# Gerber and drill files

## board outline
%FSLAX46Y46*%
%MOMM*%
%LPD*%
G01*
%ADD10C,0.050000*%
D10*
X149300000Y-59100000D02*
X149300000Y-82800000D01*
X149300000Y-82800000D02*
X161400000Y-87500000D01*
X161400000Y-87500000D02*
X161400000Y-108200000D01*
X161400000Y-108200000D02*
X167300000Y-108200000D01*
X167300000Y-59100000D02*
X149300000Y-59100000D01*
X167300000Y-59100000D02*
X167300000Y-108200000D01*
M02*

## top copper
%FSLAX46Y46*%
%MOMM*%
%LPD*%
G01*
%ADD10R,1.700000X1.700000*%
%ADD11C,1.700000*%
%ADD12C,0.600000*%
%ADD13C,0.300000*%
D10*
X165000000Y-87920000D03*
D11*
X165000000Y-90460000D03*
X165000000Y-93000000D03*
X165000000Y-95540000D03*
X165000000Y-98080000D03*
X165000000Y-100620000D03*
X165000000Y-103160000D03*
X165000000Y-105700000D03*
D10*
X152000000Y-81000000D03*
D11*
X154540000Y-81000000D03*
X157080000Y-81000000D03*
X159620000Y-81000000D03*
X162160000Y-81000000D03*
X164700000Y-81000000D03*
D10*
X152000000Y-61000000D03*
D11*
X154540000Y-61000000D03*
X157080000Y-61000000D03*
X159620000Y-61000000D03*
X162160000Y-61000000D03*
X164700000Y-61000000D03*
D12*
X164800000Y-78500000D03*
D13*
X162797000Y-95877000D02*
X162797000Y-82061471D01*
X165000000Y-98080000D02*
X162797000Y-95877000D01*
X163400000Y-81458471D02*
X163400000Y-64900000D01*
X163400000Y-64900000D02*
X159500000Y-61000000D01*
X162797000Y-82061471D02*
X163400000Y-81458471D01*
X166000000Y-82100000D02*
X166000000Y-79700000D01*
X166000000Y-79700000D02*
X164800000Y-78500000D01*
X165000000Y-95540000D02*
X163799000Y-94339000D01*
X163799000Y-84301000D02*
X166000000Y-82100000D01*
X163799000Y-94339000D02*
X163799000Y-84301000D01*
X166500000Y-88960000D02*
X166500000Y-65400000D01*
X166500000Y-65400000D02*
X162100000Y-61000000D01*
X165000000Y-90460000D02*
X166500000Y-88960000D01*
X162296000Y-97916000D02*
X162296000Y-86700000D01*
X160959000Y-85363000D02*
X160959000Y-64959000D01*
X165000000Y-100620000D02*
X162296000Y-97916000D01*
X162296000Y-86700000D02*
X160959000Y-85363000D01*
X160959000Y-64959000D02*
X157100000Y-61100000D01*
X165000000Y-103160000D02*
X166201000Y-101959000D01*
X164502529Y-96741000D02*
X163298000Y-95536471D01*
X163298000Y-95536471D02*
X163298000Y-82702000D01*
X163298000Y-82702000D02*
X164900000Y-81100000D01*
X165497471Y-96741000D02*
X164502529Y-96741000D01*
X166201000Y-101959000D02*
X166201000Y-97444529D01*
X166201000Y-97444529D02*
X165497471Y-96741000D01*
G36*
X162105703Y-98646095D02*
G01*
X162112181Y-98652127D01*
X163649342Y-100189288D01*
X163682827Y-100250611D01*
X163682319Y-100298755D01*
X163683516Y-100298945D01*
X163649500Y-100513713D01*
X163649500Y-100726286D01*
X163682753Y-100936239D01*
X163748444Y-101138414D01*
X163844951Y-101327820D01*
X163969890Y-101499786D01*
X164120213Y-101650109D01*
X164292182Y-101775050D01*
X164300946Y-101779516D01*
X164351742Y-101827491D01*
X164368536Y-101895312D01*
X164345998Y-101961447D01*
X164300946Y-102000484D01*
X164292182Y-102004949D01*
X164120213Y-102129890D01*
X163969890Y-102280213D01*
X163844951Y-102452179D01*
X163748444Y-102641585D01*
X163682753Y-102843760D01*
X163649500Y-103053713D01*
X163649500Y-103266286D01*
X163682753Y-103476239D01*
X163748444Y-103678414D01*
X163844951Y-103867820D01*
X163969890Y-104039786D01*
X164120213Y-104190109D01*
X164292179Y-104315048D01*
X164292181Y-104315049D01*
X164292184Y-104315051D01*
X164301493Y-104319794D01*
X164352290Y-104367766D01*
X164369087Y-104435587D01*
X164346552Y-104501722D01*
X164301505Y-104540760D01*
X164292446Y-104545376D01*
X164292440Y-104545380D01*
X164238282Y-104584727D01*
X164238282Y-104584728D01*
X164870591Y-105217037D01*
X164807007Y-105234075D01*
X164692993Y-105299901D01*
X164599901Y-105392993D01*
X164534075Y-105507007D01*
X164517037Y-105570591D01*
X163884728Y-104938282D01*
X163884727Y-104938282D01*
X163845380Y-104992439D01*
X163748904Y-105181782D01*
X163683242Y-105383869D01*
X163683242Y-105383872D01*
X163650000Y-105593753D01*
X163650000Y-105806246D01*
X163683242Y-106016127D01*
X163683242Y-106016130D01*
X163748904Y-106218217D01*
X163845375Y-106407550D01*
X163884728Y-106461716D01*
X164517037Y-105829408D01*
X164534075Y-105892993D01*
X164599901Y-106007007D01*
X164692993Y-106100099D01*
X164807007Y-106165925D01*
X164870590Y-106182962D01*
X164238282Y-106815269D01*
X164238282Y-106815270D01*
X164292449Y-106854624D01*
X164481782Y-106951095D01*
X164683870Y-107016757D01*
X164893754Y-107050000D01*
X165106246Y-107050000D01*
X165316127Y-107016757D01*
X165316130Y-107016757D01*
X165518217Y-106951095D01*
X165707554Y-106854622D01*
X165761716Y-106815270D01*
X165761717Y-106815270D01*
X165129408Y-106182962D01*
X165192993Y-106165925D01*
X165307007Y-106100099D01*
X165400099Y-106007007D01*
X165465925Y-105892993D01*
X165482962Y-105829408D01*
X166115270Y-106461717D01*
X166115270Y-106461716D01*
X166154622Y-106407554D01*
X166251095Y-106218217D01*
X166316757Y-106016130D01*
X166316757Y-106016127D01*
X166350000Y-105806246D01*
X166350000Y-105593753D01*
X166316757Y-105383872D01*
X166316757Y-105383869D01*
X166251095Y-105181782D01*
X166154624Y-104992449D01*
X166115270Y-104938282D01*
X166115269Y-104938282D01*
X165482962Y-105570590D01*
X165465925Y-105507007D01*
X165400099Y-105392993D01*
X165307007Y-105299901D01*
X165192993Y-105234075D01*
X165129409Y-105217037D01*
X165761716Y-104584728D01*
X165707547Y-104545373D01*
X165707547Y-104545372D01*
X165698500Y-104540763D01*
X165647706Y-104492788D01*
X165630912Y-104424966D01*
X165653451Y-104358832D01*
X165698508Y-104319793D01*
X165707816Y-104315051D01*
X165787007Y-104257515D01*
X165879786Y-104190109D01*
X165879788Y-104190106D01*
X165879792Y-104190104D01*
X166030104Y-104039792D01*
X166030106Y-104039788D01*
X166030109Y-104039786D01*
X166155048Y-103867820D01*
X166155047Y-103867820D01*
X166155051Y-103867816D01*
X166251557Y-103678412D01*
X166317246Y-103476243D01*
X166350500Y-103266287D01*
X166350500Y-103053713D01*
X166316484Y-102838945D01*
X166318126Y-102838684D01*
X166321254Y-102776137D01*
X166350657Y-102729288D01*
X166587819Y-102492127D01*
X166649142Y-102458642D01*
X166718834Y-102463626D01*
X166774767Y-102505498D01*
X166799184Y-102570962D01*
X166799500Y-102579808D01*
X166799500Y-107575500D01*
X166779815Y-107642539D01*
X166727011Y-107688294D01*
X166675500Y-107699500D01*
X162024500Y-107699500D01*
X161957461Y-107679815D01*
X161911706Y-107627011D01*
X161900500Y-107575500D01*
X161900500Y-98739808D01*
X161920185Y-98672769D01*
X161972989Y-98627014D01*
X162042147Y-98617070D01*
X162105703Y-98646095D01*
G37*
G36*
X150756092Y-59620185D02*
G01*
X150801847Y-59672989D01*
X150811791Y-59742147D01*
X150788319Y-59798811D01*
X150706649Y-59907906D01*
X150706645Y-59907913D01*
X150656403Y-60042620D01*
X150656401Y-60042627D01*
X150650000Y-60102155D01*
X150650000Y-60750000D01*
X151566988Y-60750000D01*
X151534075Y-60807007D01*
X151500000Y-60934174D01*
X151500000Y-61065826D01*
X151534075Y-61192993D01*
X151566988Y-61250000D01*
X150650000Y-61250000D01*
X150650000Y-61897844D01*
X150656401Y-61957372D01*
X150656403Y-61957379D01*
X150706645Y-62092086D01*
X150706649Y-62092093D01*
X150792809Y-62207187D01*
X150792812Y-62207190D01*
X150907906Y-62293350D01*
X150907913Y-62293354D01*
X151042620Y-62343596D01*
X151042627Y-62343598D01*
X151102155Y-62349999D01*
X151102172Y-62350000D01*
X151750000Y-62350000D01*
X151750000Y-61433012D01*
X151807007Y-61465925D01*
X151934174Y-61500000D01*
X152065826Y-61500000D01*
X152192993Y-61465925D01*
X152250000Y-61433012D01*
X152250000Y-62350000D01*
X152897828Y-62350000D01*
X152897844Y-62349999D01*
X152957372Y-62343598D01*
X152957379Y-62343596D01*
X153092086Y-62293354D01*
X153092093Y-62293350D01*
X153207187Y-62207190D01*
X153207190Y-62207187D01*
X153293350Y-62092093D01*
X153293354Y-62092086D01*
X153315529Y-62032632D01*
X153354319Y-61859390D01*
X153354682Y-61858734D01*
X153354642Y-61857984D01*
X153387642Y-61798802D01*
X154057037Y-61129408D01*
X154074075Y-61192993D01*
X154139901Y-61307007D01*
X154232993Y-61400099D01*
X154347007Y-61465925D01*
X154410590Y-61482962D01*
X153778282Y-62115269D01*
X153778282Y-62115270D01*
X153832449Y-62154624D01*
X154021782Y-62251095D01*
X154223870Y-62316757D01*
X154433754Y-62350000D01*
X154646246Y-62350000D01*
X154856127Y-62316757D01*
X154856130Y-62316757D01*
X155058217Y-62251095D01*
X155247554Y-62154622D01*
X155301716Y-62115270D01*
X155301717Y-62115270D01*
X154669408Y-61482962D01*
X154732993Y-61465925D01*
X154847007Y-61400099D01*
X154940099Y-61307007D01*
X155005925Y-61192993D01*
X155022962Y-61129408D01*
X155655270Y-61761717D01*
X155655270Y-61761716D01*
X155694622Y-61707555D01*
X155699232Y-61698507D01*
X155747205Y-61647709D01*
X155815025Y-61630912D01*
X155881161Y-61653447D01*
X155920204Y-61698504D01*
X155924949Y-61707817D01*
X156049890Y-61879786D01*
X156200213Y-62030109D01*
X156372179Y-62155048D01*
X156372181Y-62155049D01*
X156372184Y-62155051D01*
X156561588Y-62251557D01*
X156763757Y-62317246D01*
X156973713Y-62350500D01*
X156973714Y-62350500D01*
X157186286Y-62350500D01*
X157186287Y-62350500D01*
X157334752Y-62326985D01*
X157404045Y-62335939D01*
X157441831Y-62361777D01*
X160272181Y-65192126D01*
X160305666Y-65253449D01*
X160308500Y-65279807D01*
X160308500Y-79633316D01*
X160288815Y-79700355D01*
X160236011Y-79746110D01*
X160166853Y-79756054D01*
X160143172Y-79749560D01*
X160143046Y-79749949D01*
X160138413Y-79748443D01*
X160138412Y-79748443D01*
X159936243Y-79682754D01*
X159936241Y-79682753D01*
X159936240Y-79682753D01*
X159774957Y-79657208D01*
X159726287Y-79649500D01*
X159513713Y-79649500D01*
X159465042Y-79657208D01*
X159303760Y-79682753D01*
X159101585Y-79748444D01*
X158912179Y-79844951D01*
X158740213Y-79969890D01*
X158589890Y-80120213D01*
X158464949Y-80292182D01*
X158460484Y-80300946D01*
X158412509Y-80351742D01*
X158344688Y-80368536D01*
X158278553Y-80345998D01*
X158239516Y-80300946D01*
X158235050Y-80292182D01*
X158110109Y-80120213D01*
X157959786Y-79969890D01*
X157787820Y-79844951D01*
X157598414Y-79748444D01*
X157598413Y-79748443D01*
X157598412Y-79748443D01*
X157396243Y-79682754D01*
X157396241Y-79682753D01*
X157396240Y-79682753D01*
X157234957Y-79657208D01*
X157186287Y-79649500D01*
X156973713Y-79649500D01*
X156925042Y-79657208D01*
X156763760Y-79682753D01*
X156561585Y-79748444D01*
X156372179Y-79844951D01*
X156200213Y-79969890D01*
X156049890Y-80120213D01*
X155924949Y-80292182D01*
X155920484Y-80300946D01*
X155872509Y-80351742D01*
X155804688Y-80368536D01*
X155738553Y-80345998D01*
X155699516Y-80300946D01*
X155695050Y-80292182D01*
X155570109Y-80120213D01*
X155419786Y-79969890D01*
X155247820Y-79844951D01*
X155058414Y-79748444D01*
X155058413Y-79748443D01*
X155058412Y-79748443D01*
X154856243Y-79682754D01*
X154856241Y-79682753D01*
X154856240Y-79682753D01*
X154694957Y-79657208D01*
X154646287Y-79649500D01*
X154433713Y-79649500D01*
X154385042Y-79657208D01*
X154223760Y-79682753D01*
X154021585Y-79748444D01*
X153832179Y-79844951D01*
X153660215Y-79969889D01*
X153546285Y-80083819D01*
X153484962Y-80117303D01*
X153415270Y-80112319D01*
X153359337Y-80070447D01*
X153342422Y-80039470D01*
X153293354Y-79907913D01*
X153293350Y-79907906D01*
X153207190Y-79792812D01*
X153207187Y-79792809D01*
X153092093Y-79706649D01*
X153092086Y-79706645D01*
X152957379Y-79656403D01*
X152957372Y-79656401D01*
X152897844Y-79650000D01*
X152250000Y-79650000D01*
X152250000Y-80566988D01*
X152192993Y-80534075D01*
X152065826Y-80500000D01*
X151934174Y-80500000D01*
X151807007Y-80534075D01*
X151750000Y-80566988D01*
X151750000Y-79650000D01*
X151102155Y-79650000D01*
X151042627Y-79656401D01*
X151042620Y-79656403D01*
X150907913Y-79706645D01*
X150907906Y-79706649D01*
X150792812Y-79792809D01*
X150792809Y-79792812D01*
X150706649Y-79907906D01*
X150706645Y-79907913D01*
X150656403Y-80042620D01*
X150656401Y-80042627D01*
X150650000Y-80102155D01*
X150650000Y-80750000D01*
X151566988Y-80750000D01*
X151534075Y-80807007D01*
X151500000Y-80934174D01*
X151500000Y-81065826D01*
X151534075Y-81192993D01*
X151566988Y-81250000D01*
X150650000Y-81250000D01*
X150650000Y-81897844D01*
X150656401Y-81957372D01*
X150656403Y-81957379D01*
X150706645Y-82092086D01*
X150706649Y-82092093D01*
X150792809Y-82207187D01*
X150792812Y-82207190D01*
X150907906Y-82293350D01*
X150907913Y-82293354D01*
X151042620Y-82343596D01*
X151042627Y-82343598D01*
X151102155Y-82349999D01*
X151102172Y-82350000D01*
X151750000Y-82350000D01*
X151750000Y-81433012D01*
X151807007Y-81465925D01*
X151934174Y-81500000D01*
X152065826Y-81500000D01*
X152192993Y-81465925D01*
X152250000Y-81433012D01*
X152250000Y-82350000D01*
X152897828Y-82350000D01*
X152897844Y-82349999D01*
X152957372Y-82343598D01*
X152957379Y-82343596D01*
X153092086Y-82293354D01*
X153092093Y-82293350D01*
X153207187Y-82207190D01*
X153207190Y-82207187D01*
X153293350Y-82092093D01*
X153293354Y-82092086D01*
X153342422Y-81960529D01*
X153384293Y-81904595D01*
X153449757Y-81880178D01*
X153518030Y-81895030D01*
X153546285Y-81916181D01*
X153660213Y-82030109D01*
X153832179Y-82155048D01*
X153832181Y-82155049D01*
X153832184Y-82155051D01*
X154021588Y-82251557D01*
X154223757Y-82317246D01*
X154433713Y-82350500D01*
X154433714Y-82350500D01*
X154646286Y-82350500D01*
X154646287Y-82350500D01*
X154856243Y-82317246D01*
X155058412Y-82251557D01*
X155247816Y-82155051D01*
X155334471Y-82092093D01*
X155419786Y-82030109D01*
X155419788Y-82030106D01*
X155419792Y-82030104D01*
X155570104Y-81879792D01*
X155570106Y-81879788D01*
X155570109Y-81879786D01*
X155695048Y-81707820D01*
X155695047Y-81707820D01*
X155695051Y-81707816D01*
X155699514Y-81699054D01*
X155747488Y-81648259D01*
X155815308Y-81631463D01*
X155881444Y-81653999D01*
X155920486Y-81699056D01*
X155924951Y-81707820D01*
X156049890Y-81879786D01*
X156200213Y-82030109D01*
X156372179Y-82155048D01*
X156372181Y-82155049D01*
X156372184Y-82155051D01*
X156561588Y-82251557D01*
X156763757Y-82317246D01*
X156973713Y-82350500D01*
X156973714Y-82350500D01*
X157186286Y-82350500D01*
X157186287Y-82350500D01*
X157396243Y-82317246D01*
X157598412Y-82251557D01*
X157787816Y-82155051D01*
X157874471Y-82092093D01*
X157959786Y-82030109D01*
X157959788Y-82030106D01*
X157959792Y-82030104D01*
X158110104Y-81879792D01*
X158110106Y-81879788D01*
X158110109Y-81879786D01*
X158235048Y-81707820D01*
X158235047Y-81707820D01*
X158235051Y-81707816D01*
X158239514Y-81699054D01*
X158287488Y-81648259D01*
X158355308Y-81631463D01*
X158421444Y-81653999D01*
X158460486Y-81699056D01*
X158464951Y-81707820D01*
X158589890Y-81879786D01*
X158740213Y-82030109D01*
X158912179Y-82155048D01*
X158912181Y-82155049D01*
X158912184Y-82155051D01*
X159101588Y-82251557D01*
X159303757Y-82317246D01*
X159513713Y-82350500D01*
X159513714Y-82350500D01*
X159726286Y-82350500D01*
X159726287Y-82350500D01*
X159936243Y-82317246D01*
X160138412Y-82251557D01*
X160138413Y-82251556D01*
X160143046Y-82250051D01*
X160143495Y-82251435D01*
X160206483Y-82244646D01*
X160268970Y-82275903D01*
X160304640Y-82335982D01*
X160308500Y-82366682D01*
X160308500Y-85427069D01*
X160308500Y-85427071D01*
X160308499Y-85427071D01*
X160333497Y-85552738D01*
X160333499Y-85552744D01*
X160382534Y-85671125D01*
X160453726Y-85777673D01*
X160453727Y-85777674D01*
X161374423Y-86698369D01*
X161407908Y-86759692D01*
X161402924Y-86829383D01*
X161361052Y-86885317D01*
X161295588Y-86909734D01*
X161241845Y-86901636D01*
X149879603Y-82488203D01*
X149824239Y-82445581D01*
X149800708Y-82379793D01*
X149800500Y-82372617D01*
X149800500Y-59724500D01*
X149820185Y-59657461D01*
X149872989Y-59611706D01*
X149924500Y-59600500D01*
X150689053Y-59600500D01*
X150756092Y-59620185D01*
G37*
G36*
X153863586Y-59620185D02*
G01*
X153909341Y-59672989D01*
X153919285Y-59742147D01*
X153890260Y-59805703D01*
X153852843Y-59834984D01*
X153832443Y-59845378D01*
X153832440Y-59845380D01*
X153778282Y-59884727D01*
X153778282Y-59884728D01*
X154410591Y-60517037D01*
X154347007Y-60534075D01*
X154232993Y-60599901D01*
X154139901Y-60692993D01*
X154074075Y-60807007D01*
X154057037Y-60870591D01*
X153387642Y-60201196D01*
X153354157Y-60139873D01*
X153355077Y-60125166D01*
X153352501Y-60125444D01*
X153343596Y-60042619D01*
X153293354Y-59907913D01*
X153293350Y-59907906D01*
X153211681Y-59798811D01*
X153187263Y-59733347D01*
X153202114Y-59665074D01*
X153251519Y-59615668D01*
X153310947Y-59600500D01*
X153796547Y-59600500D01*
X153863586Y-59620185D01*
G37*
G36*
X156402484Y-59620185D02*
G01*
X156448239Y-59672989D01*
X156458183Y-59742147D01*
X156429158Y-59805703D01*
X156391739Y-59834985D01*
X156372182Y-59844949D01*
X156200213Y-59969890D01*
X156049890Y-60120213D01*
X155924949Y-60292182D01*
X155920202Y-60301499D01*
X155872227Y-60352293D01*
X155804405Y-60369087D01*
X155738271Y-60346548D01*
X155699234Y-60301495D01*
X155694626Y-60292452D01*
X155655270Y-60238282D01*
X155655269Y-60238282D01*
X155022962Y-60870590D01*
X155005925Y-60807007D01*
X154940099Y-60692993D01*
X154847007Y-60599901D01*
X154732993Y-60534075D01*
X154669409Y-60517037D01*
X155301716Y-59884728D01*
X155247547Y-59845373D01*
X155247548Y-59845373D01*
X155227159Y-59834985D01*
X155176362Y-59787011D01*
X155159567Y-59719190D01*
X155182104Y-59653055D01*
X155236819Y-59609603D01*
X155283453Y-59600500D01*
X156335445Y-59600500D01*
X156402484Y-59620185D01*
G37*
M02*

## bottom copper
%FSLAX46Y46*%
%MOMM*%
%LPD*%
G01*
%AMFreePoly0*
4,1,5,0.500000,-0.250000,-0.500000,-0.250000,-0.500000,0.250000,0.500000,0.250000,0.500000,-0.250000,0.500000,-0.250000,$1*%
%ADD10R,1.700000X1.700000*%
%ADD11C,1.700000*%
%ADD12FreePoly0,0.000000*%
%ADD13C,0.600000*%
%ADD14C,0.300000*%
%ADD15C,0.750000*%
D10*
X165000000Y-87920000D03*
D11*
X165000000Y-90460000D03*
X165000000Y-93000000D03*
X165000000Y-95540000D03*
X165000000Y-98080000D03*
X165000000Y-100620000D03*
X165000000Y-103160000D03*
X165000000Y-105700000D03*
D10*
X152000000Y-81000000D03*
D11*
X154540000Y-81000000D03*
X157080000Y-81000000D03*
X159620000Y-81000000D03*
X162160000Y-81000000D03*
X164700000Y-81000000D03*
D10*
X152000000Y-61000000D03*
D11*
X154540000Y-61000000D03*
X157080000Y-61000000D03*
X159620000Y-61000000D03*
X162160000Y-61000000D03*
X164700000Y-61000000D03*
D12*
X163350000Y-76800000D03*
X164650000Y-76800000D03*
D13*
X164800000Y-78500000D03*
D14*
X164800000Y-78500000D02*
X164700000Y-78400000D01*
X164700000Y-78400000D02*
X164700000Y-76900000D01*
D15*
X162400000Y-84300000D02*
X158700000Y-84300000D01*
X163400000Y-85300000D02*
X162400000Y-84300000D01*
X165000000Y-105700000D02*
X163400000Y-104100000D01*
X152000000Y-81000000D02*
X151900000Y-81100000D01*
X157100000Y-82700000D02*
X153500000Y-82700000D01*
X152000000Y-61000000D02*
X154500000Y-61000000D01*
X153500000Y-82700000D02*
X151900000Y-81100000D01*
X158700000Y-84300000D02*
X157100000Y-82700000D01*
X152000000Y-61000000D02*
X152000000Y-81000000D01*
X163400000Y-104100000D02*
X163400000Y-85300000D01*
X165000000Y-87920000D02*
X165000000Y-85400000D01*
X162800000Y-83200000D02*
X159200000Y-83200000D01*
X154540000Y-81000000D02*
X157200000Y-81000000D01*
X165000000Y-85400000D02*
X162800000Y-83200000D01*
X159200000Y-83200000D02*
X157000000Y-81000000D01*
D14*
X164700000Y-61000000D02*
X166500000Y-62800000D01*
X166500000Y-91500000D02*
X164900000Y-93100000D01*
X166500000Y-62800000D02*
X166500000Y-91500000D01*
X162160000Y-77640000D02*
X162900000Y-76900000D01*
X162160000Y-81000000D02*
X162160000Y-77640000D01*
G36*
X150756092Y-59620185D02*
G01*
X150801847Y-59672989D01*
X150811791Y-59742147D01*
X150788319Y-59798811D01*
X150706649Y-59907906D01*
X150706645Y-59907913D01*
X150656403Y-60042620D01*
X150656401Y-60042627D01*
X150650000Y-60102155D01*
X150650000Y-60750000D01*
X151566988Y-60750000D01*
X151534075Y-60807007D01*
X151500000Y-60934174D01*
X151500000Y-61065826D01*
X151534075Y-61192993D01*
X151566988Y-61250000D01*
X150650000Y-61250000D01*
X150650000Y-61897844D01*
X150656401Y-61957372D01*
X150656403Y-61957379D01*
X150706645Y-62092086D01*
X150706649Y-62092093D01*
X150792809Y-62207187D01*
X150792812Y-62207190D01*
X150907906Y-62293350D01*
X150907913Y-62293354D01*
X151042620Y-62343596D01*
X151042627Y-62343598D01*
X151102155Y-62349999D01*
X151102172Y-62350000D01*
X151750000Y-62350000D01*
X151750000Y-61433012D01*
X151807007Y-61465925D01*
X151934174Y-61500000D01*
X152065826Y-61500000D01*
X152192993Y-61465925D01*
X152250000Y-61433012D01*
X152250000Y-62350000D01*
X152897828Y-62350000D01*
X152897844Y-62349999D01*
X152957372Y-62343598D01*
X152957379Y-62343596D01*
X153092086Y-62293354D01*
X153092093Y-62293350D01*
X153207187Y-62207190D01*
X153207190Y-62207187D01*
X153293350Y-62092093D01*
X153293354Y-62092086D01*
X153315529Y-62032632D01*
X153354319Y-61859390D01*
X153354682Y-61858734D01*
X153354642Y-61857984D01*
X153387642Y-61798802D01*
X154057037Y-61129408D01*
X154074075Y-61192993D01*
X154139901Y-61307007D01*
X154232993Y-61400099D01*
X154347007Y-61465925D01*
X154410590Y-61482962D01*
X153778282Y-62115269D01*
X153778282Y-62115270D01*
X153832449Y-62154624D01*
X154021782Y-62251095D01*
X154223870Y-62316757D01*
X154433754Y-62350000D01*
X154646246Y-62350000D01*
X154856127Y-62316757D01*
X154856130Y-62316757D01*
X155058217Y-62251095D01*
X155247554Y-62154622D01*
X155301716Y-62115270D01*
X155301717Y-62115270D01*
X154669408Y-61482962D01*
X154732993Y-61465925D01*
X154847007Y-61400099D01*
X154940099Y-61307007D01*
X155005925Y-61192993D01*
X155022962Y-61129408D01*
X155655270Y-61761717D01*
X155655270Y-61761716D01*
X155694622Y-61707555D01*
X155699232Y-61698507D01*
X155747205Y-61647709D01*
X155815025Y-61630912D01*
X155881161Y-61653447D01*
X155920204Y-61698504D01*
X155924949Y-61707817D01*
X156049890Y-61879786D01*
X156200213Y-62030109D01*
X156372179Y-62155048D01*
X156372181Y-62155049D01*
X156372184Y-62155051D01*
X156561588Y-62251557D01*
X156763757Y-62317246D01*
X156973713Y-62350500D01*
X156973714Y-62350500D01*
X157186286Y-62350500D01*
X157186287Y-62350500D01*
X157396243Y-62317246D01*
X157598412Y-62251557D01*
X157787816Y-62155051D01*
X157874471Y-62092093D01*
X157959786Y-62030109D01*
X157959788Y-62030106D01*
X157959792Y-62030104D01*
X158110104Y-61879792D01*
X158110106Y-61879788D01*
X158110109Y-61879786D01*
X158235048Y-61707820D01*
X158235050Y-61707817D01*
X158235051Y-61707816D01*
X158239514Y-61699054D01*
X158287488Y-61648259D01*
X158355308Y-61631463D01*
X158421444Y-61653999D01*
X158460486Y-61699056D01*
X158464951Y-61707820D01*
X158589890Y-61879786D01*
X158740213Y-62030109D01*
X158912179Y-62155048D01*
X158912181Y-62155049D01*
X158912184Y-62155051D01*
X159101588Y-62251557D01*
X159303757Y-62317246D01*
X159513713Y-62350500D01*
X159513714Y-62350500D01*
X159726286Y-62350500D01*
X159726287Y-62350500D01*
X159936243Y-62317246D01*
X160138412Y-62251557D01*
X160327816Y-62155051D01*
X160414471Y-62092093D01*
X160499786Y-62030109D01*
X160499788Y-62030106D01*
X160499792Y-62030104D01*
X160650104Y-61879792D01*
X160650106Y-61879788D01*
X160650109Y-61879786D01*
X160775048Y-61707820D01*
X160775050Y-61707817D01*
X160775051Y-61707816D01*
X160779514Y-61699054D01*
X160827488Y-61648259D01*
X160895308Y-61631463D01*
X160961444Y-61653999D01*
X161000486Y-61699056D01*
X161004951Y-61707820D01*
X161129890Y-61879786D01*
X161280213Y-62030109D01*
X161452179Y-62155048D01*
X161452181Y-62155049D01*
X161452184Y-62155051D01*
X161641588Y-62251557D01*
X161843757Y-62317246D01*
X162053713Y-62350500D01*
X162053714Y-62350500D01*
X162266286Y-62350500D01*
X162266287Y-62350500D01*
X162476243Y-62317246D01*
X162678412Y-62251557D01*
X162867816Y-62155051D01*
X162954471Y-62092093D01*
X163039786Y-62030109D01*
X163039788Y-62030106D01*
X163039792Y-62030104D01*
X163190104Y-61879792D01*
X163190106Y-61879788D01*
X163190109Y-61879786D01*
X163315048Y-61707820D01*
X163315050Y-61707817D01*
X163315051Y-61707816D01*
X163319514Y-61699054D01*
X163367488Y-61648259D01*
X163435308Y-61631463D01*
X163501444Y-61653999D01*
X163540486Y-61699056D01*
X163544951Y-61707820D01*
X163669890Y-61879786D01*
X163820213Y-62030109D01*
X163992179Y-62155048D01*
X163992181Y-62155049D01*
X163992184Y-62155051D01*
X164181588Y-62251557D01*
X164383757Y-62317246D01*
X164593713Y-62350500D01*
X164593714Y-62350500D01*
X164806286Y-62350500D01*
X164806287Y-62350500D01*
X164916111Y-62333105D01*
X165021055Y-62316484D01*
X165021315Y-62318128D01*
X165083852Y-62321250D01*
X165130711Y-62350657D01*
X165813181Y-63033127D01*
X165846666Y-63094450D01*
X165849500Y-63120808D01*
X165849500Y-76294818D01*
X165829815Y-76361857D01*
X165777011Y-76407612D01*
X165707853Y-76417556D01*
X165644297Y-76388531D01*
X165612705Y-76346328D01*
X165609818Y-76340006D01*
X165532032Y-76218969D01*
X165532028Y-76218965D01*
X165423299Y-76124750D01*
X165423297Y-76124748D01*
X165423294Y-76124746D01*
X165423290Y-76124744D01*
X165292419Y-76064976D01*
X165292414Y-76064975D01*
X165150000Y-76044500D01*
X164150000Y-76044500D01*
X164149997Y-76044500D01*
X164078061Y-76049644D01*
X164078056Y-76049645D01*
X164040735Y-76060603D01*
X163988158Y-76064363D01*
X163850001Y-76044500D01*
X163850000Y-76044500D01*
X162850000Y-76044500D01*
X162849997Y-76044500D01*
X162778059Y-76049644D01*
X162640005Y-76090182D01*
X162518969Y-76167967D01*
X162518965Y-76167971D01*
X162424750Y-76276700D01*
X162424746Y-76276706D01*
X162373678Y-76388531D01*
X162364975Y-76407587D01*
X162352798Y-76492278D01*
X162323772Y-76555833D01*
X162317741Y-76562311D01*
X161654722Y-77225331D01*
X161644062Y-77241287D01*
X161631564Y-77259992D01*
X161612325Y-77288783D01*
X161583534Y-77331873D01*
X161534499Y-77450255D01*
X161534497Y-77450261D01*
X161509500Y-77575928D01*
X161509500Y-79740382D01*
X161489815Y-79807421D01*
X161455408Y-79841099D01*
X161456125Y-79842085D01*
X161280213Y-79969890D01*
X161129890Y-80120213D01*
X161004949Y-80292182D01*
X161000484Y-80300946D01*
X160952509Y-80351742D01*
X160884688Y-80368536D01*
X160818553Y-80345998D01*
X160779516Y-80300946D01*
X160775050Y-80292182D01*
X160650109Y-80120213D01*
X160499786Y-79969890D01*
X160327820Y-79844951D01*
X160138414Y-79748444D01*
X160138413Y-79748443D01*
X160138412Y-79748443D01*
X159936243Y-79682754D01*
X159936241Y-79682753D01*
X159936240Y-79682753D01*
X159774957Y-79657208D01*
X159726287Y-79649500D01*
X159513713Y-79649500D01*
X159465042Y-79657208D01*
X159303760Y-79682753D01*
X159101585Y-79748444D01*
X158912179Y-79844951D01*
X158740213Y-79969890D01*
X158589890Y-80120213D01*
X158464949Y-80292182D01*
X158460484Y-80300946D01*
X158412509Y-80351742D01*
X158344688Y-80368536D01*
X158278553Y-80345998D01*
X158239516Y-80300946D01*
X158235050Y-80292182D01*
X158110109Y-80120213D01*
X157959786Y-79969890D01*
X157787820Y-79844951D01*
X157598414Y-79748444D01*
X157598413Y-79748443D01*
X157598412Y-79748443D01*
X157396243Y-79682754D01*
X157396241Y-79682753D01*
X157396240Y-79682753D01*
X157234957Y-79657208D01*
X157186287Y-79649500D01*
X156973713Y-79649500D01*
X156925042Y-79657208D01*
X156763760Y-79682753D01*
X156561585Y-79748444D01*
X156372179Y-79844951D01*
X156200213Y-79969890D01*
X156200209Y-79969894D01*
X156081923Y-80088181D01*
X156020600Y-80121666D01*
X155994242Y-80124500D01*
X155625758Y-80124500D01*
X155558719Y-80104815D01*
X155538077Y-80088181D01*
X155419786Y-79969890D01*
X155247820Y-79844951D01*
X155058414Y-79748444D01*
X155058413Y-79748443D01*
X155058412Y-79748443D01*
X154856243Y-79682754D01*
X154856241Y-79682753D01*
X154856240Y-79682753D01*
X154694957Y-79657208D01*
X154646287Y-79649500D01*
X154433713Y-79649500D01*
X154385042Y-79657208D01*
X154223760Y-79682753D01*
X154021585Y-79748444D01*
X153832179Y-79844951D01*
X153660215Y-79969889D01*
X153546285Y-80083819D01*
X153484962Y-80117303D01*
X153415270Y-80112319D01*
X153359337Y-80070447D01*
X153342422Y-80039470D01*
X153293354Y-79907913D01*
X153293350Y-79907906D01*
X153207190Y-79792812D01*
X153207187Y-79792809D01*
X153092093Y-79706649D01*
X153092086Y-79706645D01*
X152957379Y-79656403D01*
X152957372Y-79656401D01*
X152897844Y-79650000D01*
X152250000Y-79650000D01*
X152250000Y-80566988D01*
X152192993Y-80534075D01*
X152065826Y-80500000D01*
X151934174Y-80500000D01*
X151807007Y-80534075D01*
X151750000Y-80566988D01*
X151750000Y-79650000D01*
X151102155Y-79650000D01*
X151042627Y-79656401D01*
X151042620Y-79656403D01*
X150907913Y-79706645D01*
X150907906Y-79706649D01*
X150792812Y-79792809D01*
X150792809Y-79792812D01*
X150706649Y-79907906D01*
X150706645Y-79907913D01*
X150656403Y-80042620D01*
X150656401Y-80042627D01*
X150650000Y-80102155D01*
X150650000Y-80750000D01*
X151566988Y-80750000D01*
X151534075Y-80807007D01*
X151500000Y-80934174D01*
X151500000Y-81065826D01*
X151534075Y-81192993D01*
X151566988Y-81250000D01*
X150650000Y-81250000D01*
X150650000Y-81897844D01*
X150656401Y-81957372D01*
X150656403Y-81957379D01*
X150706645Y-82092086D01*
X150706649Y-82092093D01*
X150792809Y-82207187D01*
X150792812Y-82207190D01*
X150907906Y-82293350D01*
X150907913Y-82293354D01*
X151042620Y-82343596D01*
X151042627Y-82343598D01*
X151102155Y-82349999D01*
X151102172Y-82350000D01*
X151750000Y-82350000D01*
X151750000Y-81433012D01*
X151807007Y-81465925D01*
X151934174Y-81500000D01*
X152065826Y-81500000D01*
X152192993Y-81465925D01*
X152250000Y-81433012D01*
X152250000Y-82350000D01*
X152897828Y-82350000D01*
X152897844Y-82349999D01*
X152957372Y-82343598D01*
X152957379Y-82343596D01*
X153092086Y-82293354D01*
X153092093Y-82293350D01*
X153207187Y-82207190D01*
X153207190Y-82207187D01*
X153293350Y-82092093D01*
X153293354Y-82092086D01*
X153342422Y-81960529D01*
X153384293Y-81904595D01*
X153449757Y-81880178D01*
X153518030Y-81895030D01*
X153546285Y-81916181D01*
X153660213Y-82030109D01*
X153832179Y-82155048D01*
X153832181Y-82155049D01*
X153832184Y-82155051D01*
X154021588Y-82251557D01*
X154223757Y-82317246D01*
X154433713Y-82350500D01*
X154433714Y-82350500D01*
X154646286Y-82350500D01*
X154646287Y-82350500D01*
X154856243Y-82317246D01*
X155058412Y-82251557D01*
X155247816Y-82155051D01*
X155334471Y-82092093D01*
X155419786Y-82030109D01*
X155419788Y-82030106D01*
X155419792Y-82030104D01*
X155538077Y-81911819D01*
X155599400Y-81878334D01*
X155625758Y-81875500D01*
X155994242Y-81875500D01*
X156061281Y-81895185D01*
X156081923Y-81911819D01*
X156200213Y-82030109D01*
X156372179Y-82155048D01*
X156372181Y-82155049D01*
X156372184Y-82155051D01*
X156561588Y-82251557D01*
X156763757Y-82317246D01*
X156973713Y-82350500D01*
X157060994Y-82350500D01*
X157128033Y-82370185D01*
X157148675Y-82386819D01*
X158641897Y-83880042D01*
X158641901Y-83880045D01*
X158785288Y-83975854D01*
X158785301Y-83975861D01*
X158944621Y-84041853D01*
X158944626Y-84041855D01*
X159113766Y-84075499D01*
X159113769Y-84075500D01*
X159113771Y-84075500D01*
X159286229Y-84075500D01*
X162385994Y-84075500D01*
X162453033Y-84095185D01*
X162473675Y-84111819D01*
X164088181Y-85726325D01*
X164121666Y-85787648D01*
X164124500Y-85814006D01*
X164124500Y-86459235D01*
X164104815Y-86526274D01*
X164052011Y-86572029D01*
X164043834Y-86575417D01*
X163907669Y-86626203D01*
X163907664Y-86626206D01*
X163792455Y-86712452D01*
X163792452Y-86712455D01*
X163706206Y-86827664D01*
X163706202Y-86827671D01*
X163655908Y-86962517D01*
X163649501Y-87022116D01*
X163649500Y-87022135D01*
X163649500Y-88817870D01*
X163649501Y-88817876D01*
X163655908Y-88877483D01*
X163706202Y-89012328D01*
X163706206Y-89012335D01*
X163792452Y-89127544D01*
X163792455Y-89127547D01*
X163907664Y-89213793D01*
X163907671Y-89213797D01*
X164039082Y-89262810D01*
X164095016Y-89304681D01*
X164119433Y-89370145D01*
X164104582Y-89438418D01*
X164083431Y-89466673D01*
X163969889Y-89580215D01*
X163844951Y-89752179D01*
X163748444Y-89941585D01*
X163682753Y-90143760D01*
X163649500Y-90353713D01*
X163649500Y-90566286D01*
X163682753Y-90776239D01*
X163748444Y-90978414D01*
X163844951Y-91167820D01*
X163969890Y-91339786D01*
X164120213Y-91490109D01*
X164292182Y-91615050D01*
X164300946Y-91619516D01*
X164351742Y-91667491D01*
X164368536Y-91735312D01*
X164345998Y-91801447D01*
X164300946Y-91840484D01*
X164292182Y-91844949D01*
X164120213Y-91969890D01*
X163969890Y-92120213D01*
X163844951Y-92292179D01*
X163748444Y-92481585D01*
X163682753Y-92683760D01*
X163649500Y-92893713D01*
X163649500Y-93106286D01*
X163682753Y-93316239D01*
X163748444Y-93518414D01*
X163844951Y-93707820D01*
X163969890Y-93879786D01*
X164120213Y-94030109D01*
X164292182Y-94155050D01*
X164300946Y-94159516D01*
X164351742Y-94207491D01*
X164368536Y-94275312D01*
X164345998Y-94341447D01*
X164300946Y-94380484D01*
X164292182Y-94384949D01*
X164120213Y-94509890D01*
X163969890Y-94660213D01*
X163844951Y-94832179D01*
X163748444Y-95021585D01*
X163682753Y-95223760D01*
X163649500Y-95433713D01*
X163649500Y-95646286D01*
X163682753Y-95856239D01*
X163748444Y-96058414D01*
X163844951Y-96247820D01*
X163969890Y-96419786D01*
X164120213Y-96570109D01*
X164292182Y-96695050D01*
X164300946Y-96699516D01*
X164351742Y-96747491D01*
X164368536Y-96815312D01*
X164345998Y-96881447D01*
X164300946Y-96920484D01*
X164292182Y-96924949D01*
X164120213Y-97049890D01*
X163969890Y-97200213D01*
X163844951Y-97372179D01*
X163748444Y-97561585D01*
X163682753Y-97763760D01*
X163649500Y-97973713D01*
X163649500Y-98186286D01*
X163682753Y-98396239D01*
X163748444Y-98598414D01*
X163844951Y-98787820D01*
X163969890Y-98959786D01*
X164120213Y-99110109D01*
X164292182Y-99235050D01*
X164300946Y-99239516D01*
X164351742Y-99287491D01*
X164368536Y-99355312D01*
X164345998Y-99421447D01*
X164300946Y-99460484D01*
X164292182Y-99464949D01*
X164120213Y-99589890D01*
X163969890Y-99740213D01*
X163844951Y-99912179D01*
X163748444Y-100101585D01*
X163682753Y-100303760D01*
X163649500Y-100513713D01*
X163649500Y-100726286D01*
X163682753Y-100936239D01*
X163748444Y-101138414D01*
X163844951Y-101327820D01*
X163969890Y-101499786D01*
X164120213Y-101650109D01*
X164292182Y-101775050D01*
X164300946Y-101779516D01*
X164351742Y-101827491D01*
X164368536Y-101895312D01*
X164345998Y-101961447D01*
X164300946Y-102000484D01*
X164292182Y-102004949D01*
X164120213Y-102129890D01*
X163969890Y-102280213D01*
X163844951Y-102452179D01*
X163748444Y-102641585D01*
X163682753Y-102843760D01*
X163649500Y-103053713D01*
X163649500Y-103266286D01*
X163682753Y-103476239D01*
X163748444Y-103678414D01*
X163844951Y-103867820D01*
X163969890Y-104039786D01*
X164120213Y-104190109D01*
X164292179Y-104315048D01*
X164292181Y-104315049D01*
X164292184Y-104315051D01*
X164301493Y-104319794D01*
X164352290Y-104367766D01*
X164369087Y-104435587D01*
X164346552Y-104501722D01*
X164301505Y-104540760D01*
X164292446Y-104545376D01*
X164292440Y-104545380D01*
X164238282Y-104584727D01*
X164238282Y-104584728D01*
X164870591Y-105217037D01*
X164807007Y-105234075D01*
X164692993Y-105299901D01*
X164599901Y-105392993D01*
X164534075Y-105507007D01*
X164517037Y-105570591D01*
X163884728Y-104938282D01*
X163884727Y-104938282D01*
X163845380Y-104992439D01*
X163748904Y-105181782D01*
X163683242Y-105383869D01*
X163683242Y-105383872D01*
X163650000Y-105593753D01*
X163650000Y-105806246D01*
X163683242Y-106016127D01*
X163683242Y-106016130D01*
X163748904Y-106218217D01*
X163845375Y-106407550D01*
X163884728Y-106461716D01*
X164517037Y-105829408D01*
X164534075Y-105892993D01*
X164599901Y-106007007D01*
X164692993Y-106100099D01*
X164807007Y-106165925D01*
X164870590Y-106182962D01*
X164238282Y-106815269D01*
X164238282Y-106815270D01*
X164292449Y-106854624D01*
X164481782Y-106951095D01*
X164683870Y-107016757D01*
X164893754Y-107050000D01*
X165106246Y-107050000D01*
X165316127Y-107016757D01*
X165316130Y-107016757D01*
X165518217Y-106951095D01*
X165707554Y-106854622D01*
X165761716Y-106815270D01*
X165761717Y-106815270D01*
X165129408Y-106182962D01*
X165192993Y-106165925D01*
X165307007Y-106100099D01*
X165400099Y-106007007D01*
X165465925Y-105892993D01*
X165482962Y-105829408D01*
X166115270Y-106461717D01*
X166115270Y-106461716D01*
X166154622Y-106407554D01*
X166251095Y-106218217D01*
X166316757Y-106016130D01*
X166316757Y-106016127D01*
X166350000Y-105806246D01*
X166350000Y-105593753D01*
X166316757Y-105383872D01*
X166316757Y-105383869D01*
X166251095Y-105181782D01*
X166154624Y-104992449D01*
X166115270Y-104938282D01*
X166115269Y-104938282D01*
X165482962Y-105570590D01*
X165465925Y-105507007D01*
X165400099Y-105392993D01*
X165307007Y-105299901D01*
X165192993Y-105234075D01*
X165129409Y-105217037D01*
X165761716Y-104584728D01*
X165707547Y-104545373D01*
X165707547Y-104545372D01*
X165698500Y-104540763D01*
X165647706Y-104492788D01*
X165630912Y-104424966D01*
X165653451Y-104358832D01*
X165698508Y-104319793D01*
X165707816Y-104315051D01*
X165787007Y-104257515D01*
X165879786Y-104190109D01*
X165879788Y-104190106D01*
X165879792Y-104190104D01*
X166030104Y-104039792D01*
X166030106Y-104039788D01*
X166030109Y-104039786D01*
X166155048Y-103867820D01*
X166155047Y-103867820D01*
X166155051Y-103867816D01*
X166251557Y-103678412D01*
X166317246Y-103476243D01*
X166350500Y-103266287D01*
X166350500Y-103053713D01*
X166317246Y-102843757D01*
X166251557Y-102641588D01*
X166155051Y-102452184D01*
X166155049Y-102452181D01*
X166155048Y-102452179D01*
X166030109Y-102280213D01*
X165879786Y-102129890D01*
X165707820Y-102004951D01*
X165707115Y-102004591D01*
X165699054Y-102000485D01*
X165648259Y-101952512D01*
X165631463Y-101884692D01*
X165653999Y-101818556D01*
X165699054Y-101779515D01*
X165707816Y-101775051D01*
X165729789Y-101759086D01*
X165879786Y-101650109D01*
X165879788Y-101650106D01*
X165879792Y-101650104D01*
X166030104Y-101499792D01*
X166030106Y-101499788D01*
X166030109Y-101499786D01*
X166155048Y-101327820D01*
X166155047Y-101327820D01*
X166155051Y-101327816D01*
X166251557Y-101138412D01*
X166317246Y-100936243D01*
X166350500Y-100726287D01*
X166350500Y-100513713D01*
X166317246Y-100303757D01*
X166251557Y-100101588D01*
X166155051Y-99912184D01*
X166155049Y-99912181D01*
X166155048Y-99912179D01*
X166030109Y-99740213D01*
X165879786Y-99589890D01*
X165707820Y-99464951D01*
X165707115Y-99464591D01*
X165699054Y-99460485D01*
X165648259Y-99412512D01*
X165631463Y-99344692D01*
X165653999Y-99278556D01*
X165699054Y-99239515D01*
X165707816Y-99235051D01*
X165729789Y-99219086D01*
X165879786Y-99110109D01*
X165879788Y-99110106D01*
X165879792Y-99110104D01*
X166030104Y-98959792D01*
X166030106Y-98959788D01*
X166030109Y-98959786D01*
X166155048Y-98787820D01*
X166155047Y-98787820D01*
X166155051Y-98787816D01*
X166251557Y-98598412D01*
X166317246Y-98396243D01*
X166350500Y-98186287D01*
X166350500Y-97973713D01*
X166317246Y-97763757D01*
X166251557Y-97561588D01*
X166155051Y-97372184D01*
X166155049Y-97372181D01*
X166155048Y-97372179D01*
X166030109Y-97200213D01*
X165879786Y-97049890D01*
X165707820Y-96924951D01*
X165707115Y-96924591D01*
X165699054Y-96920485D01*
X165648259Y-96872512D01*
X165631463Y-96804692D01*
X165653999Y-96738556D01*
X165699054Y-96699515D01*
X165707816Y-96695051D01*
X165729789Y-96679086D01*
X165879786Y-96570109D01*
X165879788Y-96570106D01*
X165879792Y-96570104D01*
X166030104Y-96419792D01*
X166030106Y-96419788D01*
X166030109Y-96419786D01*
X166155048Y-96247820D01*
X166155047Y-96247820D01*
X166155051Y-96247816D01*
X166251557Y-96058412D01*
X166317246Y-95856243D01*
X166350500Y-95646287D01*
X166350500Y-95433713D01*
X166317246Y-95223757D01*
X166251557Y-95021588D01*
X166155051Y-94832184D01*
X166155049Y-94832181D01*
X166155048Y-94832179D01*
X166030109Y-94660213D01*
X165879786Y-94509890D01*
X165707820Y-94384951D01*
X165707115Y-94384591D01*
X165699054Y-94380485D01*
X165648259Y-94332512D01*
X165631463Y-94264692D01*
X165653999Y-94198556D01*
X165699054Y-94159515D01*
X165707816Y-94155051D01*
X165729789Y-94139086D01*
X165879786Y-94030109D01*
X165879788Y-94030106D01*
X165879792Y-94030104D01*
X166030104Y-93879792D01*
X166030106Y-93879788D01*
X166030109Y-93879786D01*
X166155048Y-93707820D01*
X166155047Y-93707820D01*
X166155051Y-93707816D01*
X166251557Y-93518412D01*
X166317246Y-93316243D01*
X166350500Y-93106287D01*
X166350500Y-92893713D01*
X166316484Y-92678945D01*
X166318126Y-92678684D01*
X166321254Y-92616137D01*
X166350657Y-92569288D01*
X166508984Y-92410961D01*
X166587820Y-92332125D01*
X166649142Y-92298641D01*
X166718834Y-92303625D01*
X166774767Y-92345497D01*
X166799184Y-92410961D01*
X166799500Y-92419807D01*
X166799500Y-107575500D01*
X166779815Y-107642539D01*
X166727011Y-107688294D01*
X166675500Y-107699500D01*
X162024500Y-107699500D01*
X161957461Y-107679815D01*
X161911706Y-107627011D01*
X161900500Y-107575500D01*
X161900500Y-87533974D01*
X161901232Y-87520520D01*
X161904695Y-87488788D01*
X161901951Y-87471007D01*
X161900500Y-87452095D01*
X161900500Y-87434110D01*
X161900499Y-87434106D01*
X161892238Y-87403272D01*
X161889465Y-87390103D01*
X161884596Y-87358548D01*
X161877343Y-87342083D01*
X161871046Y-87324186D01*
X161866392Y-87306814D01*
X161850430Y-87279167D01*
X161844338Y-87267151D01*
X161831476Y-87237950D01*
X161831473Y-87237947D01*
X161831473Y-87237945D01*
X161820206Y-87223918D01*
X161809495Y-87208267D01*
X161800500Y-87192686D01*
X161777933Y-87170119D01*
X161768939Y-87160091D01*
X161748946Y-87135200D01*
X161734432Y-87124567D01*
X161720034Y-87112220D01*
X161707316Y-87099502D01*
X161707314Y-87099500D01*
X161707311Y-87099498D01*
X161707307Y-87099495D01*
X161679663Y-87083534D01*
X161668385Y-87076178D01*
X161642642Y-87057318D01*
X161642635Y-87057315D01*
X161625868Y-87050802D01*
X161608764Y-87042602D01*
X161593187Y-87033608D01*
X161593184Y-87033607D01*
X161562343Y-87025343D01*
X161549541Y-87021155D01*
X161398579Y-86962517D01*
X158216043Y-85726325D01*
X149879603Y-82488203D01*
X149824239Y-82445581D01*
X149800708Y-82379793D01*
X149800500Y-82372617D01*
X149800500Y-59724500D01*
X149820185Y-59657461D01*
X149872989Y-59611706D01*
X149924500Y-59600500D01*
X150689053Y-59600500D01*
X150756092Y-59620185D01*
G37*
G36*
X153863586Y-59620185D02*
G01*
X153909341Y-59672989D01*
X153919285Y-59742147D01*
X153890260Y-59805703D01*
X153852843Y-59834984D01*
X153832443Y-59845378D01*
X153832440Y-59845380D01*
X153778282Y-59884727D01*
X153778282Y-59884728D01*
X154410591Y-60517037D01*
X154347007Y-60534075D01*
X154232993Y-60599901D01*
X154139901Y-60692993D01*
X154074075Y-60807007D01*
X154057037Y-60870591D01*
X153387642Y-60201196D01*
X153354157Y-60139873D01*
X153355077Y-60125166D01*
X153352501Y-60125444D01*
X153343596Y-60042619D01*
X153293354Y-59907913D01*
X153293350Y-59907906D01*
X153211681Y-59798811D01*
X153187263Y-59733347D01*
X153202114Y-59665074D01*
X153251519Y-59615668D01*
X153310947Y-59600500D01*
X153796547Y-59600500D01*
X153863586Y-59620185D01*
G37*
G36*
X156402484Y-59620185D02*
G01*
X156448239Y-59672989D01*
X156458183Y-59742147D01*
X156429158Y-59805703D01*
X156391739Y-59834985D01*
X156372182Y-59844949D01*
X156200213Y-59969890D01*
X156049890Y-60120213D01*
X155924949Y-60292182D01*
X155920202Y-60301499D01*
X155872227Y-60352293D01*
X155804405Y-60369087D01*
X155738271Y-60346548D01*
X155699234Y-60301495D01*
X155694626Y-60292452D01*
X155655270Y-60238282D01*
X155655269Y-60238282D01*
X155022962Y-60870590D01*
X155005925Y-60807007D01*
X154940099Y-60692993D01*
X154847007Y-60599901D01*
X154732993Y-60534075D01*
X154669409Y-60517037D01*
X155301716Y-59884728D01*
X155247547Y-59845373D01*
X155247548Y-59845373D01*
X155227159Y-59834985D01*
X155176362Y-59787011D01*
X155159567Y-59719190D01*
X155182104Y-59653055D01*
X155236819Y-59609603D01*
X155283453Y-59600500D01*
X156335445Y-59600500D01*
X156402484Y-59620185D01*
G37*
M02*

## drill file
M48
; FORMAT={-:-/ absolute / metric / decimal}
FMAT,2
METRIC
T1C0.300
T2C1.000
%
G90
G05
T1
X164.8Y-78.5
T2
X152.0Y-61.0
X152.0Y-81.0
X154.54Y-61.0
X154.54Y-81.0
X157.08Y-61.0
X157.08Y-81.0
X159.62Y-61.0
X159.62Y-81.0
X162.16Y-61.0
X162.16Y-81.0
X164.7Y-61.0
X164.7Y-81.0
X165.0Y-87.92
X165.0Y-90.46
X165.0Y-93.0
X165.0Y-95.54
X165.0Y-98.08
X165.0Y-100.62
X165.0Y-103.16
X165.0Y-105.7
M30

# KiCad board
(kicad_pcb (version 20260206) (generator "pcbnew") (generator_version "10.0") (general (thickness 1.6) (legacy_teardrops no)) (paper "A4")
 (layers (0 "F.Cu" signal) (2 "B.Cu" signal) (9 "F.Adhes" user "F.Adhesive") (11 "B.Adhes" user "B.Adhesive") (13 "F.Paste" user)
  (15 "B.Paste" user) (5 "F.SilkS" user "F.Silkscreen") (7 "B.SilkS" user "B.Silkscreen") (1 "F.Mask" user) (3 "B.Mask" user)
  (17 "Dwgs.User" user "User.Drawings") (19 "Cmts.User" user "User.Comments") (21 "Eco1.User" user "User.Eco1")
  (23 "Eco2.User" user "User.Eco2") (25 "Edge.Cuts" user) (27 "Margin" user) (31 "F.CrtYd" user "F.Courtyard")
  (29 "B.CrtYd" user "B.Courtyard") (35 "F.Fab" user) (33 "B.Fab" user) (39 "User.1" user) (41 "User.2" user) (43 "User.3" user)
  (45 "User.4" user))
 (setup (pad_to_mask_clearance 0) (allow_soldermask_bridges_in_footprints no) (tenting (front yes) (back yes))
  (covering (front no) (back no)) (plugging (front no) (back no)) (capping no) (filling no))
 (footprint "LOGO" (layer "F.Cu") (at 158.5 70.4)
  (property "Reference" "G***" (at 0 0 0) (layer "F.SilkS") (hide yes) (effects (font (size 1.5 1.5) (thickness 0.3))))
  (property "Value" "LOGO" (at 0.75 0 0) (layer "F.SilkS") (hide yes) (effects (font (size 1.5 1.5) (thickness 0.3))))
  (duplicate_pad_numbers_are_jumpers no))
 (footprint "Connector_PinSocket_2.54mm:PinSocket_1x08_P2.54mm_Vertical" (layer "B.Cu") (at 165 87.92 180)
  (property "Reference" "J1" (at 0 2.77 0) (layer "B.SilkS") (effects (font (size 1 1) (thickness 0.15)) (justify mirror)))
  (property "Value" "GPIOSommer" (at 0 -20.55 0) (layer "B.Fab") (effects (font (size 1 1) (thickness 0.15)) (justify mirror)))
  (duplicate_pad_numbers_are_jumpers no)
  (pad "1" thru_hole rect (at 0 0 180) (size 1.7 1.7) (drill 1) (layers "*.Cu" "*.Mask") (remove_unused_layers no) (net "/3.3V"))
  (pad "2" thru_hole circle (at 0 -2.54 180) (size 1.7 1.7) (drill 1) (layers "*.Cu" "*.Mask") (remove_unused_layers no) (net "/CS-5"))
  (pad "3" thru_hole circle (at 0 -5.08 180) (size 1.7 1.7) (drill 1) (layers "*.Cu" "*.Mask") (remove_unused_layers no) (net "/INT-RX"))
  (pad "4" thru_hole circle (at 0 -7.62 180) (size 1.7 1.7) (drill 1) (layers "*.Cu" "*.Mask") (remove_unused_layers no) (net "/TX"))
  (pad "5" thru_hole circle (at 0 -10.16 180) (size 1.7 1.7) (drill 1) (layers "*.Cu" "*.Mask") (remove_unused_layers no) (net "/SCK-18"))
  (pad "6" thru_hole circle (at 0 -12.7 180) (size 1.7 1.7) (drill 1) (layers "*.Cu" "*.Mask") (remove_unused_layers no) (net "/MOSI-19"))
  (pad "7" thru_hole circle (at 0 -15.24 180) (size 1.7 1.7) (drill 1) (layers "*.Cu" "*.Mask") (remove_unused_layers no) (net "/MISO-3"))
  (pad "8" thru_hole circle (at 0 -17.78 180) (size 1.7 1.7) (drill 1) (layers "*.Cu" "*.Mask") (remove_unused_layers no) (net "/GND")))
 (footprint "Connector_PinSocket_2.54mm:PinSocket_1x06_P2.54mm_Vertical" (layer "B.Cu") (at 152 81 -90)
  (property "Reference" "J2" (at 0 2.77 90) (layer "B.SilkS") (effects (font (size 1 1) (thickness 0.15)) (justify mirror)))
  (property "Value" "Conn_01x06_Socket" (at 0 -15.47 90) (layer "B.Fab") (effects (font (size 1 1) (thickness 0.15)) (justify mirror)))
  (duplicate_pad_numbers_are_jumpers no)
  (pad "1" thru_hole rect (at 0 0 270) (size 1.7 1.7) (drill 1) (layers "*.Cu" "*.Mask") (remove_unused_layers no) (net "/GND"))
  (pad "2" thru_hole circle (at 0 -2.54 270) (size 1.7 1.7) (drill 1) (layers "*.Cu" "*.Mask") (remove_unused_layers no) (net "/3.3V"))
  (pad "3" thru_hole circle (at 0 -5.08 270) (size 1.7 1.7) (drill 1) (layers "*.Cu" "*.Mask") (remove_unused_layers no) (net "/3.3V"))
  (pad "4" thru_hole circle (at 0 -7.62 270) (size 1.7 1.7) (drill 1) (layers "*.Cu" "*.Mask") (remove_unused_layers no)
   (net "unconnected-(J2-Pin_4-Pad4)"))
  (pad "5" thru_hole circle (at 0 -10.16 270) (size 1.7 1.7) (drill 1) (layers "*.Cu" "*.Mask") (remove_unused_layers no) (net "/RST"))
  (pad "6" thru_hole circle (at 0 -12.7 270) (size 1.7 1.7) (drill 1) (layers "*.Cu" "*.Mask") (remove_unused_layers no) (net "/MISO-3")))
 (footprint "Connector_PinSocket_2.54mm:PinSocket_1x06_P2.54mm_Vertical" (layer "B.Cu") (at 152 61 -90)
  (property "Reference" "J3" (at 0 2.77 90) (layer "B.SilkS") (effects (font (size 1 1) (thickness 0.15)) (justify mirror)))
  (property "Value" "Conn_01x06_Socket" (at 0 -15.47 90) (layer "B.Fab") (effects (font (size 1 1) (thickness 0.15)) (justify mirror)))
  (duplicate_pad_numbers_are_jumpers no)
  (pad "1" thru_hole rect (at 0 0 270) (size 1.7 1.7) (drill 1) (layers "*.Cu" "*.Mask") (remove_unused_layers no) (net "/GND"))
  (pad "2" thru_hole circle (at 0 -2.54 270) (size 1.7 1.7) (drill 1) (layers "*.Cu" "*.Mask") (remove_unused_layers no) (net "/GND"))
  (pad "3" thru_hole circle (at 0 -5.08 270) (size 1.7 1.7) (drill 1) (layers "*.Cu" "*.Mask") (remove_unused_layers no) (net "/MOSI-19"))
  (pad "4" thru_hole circle (at 0 -7.62 270) (size 1.7 1.7) (drill 1) (layers "*.Cu" "*.Mask") (remove_unused_layers no) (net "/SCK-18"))
  (pad "5" thru_hole circle (at 0 -10.16 270) (size 1.7 1.7) (drill 1) (layers "*.Cu" "*.Mask") (remove_unused_layers no) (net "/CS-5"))
  (pad "6" thru_hole circle (at 0 -12.7 270) (size 1.7 1.7) (drill 1) (layers "*.Cu" "*.Mask") (remove_unused_layers no) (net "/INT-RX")))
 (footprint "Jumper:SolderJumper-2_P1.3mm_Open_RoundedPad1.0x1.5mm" (layer "B.Cu") (at 164 76.8)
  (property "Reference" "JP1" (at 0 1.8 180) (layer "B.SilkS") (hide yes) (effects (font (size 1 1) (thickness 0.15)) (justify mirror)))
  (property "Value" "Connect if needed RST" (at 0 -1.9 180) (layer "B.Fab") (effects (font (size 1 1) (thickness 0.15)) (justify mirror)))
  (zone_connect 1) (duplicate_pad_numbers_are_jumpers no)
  (pad "1" smd custom (at -0.65 0) (size 1 0.5) (layers "B.Cu" "B.Mask") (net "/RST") (zone_connect 2) (thermal_bridge_angle 45)
   (options (clearance outline) (anchor rect)) (primitives))
  (pad "2" smd custom (at 0.65 0) (size 1 0.5) (layers "B.Cu" "B.Mask") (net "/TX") (zone_connect 2) (thermal_bridge_angle 45)
   (options (clearance outline) (anchor rect)) (primitives)))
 (gr_line (start 149.3 59.1) (end 149.3 82.8) (stroke (width 0.05) (type default)) (layer "Edge.Cuts"))
 (gr_line (start 149.3 82.8) (end 161.4 87.5) (stroke (width 0.05) (type default)) (layer "Edge.Cuts"))
 (gr_line (start 161.4 87.5) (end 161.4 108.2) (stroke (width 0.05) (type default)) (layer "Edge.Cuts"))
 (gr_line (start 161.4 108.2) (end 167.3 108.2) (stroke (width 0.05) (type default)) (layer "Edge.Cuts"))
 (gr_line (start 167.3 59.1) (end 149.3 59.1) (stroke (width 0.05) (type default)) (layer "Edge.Cuts"))
 (gr_line (start 167.3 59.1) (end 167.3 108.2) (stroke (width 0.05) (type default)) (layer "Edge.Cuts"))
 (segment (start 162.797 95.877) (end 162.797 82.061471) (width 0.3) (layer "F.Cu") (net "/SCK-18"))
 (segment (start 165 98.08) (end 162.797 95.877) (width 0.3) (layer "F.Cu") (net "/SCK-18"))
 (segment (start 163.4 81.458471) (end 163.4 64.9) (width 0.3) (layer "F.Cu") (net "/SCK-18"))
 (segment (start 163.4 64.9) (end 159.5 61) (width 0.3) (layer "F.Cu") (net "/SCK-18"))
 (segment (start 162.797 82.061471) (end 163.4 81.458471) (width 0.3) (layer "F.Cu") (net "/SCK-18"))
 (segment (start 166 82.1) (end 166 79.7) (width 0.3) (layer "F.Cu") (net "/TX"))
 (segment (start 166 79.7) (end 164.8 78.5) (width 0.3) (layer "F.Cu") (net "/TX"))
 (segment (start 165 95.54) (end 163.799 94.339) (width 0.3) (layer "F.Cu") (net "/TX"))
 (segment (start 163.799 84.301) (end 166 82.1) (width 0.3) (layer "F.Cu") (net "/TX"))
 (segment (start 163.799 94.339) (end 163.799 84.301) (width 0.3) (layer "F.Cu") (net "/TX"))
 (via (at 164.8 78.5) (size 0.6) (drill 0.3) (layers "F.Cu" "B.Cu") (capping no) (covering (front no) (back no))
  (plugging (front no) (back no)) (filling no) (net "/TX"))
 (segment (start 164.8 78.5) (end 164.7 78.4) (width 0.3) (layer "B.Cu") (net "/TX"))
 (segment (start 164.7 78.4) (end 164.7 76.9) (width 0.3) (layer "B.Cu") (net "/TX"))
 (segment (start 162.4 84.3) (end 158.7 84.3) (width 0.75) (layer "B.Cu") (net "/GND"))
 (segment (start 163.4 85.3) (end 162.4 84.3) (width 0.75) (layer "B.Cu") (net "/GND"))
 (segment (start 165 105.7) (end 163.4 104.1) (width 0.75) (layer "B.Cu") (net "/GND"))
 (segment (start 152 81) (end 151.9 81.1) (width 0.75) (layer "B.Cu") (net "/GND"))
 (segment (start 157.1 82.7) (end 153.5 82.7) (width 0.75) (layer "B.Cu") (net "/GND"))
 (segment (start 152 61) (end 154.5 61) (width 0.75) (layer "B.Cu") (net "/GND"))
 (segment (start 153.5 82.7) (end 151.9 81.1) (width 0.75) (layer "B.Cu") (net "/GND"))
 (segment (start 158.7 84.3) (end 157.1 82.7) (width 0.75) (layer "B.Cu") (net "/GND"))
 (segment (start 152 61) (end 152 81) (width 0.75) (layer "B.Cu") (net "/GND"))
 (segment (start 163.4 104.1) (end 163.4 85.3) (width 0.75) (layer "B.Cu") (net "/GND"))
 (segment (start 166.5 88.96) (end 166.5 65.4) (width 0.3) (layer "F.Cu") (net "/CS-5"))
 (segment (start 166.5 65.4) (end 162.1 61) (width 0.3) (layer "F.Cu") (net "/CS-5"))
 (segment (start 165 90.46) (end 166.5 88.96) (width 0.3) (layer "F.Cu") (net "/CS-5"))
 (segment (start 162.296 97.916) (end 162.296 86.7) (width 0.3) (layer "F.Cu") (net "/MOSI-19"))
 (segment (start 160.959 85.363) (end 160.959 64.959) (width 0.3) (layer "F.Cu") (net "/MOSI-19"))
 (segment (start 165 100.62) (end 162.296 97.916) (width 0.3) (layer "F.Cu") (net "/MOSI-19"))
 (segment (start 162.296 86.7) (end 160.959 85.363) (width 0.3) (layer "F.Cu") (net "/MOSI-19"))
 (segment (start 160.959 64.959) (end 157.1 61.1) (width 0.3) (layer "F.Cu") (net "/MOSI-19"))
 (segment (start 165 103.16) (end 166.201 101.959) (width 0.3) (layer "F.Cu") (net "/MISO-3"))
 (segment (start 164.502529 96.741) (end 163.298 95.536471) (width 0.3) (layer "F.Cu") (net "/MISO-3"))
 (segment (start 163.298 95.536471) (end 163.298 82.702) (width 0.3) (layer "F.Cu") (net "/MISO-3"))
 (segment (start 163.298 82.702) (end 164.9 81.1) (width 0.3) (layer "F.Cu") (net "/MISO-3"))
 (segment (start 165.497471 96.741) (end 164.502529 96.741) (width 0.3) (layer "F.Cu") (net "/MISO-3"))
 (segment (start 166.201 101.959) (end 166.201 97.444529) (width 0.3) (layer "F.Cu") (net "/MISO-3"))
 (segment (start 166.201 97.444529) (end 165.497471 96.741) (width 0.3) (layer "F.Cu") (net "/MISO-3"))
 (segment (start 165 87.92) (end 165 85.4) (width 0.75) (layer "B.Cu") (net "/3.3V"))
 (segment (start 162.8 83.2) (end 159.2 83.2) (width 0.75) (layer "B.Cu") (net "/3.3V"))
 (segment (start 154.54 81) (end 157.2 81) (width 0.75) (layer "B.Cu") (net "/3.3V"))
 (segment (start 165 85.4) (end 162.8 83.2) (width 0.75) (layer "B.Cu") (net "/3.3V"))
 (segment (start 159.2 83.2) (end 157 81) (width 0.75) (layer "B.Cu") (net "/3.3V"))
 (segment (start 164.7 61) (end 166.5 62.8) (width 0.3) (layer "B.Cu") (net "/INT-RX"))
 (segment (start 166.5 91.5) (end 164.9 93.1) (width 0.3) (layer "B.Cu") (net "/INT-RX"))
 (segment (start 166.5 62.8) (end 166.5 91.5) (width 0.3) (layer "B.Cu") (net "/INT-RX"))
 (segment (start 162.16 77.64) (end 162.9 76.9) (width 0.3) (layer "B.Cu") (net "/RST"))
 (segment (start 162.16 81) (end 162.16 77.64) (width 0.3) (layer "B.Cu") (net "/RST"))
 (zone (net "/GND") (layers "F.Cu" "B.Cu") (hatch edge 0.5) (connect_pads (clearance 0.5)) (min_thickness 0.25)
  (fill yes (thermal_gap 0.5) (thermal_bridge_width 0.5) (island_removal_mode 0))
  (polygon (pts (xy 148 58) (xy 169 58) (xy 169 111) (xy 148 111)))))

